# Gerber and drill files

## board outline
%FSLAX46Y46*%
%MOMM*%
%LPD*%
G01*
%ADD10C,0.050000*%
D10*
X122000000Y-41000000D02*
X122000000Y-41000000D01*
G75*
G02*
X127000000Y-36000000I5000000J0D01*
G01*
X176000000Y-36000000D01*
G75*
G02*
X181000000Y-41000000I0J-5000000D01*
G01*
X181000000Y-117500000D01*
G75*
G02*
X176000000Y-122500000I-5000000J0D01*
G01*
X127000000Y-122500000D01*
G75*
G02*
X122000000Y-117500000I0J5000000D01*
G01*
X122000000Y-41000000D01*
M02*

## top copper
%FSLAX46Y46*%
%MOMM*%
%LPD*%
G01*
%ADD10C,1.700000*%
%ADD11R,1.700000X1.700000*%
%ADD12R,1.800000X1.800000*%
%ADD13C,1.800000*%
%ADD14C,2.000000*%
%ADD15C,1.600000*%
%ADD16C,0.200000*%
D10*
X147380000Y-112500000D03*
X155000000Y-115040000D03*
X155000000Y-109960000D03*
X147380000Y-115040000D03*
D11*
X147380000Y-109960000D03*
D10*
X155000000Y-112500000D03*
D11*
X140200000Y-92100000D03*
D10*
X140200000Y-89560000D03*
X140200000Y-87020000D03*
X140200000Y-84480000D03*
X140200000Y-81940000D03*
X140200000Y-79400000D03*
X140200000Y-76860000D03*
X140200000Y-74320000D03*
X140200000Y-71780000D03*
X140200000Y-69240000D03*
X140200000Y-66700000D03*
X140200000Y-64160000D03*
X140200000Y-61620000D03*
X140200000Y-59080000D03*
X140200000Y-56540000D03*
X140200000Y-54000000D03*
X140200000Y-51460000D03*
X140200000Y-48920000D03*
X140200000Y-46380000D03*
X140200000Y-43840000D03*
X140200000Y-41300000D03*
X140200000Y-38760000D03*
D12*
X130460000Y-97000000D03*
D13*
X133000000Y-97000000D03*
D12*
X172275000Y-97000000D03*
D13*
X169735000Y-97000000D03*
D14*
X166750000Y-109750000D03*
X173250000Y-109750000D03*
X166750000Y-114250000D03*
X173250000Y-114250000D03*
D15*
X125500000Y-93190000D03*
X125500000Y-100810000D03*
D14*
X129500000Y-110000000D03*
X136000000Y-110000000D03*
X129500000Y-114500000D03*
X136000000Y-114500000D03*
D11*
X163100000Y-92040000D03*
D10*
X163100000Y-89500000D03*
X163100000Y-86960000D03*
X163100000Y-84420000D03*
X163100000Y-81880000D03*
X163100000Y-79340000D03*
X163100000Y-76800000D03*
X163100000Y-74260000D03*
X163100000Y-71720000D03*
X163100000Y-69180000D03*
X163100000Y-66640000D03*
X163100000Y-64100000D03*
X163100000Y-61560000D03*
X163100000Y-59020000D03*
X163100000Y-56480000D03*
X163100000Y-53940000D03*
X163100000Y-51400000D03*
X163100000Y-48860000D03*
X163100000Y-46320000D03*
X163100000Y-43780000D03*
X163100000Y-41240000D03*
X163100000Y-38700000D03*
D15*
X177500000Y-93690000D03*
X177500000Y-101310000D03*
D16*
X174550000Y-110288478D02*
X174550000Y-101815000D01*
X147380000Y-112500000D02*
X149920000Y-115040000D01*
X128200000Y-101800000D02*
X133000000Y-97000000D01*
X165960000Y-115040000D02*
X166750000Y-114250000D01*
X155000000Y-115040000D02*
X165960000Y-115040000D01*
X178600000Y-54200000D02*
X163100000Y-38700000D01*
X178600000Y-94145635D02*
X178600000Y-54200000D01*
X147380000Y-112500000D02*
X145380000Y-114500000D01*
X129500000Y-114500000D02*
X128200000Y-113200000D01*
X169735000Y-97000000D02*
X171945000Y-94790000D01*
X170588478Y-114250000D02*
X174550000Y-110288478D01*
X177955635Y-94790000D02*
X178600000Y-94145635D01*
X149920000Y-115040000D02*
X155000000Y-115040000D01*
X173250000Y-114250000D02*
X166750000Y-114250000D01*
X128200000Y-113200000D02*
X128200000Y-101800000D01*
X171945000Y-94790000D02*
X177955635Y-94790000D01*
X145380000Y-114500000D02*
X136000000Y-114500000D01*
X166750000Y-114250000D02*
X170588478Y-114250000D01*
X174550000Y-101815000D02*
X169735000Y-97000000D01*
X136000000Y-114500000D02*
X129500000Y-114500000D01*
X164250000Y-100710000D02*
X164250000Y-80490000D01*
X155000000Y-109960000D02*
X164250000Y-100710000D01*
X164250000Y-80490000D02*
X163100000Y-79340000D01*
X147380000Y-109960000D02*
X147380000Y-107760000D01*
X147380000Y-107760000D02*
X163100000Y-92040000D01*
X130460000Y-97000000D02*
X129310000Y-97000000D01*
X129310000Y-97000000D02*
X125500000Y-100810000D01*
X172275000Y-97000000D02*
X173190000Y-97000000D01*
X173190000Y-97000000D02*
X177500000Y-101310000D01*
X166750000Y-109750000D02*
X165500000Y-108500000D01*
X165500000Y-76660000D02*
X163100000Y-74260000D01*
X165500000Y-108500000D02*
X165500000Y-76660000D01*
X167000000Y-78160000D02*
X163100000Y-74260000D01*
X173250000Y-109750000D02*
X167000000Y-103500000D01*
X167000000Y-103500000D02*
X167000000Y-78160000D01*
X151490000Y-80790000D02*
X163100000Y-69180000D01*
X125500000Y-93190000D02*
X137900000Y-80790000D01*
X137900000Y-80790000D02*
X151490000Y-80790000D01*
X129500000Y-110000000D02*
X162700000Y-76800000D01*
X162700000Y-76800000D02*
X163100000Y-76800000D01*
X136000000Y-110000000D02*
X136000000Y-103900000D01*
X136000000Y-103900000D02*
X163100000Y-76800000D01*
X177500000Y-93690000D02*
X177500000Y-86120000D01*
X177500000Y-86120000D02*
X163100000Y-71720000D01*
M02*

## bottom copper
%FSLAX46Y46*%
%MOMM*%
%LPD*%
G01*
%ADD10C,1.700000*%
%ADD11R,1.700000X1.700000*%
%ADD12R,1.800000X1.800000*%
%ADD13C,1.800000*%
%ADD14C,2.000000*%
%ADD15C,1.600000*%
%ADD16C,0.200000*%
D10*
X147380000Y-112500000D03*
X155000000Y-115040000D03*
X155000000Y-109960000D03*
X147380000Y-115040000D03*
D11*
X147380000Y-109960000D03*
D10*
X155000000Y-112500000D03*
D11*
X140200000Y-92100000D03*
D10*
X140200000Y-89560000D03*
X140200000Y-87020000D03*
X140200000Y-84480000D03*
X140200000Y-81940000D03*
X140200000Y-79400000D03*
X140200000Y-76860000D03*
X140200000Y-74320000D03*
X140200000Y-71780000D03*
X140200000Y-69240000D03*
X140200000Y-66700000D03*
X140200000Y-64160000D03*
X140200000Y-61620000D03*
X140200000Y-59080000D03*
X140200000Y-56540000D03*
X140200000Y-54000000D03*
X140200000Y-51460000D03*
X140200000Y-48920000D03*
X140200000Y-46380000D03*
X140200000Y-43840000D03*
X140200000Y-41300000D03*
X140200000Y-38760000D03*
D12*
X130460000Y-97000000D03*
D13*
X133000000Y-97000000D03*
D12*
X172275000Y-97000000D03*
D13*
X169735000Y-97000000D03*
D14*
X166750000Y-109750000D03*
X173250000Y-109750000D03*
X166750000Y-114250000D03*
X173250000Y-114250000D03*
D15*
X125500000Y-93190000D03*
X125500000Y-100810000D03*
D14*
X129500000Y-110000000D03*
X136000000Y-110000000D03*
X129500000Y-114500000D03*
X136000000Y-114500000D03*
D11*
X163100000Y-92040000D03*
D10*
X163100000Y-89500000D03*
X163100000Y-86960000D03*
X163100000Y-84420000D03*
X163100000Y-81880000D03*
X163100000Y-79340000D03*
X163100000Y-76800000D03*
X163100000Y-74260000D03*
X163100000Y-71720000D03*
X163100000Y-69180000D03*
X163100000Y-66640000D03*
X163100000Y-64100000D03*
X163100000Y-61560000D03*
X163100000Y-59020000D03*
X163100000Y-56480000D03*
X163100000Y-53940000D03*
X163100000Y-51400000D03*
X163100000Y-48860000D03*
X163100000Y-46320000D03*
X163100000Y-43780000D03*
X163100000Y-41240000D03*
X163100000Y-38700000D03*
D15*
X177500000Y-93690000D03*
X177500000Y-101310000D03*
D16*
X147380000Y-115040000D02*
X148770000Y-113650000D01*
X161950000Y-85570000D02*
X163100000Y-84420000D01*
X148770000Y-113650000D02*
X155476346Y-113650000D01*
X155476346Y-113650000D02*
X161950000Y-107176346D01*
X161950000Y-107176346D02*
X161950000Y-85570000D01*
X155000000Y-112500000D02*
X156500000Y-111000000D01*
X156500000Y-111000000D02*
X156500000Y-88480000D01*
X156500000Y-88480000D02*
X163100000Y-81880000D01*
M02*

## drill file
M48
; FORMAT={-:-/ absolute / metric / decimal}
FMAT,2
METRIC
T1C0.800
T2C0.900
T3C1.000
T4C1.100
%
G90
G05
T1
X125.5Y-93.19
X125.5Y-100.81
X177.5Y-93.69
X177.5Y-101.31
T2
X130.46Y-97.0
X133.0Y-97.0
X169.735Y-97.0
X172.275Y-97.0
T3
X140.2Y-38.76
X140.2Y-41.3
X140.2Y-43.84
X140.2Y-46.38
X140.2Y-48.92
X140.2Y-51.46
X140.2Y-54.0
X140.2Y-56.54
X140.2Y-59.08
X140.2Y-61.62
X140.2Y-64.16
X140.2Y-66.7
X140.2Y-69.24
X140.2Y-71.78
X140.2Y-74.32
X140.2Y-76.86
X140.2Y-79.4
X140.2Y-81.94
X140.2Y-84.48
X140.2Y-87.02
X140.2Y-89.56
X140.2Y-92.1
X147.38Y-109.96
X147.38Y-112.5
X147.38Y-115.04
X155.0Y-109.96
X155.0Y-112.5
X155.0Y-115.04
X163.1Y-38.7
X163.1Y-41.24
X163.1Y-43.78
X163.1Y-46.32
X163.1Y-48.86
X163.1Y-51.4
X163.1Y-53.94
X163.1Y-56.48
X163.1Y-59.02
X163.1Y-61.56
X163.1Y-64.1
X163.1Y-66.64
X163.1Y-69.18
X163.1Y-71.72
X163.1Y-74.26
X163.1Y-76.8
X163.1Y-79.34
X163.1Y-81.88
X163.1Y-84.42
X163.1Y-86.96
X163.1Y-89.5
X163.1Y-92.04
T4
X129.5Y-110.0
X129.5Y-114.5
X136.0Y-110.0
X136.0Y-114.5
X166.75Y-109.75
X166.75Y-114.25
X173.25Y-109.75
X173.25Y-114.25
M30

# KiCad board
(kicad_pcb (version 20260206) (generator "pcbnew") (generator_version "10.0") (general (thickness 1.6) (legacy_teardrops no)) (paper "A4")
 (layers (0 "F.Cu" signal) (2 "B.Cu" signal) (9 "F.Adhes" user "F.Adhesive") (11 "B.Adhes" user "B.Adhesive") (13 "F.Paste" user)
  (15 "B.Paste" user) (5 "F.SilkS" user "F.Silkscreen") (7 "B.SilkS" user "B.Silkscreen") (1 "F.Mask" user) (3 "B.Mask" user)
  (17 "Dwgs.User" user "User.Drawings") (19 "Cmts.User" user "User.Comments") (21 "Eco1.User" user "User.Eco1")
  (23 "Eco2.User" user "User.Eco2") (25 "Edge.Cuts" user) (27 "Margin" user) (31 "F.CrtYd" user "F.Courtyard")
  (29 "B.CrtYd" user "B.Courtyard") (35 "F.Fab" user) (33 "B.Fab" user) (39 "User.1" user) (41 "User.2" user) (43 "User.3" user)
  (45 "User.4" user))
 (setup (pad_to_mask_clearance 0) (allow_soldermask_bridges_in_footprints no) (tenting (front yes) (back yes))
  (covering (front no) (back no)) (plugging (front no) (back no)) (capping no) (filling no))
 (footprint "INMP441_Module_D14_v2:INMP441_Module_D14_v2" (layer "F.Cu") (at 151.19 112.5)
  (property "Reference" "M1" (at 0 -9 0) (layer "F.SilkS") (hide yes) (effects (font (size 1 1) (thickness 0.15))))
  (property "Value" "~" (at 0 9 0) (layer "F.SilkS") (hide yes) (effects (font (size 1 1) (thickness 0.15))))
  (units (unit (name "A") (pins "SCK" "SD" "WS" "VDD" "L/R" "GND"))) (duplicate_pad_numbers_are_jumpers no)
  (pad "GND" thru_hole circle (at -3.81 0) (size 1.7 1.7) (drill 1) (layers "*.Cu" "*.Mask" "F.SilkS") (remove_unused_layers no) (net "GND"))
  (pad "L/R" thru_hole circle (at 3.81 2.54) (size 1.7 1.7) (drill 1) (layers "*.Cu" "*.Mask" "F.SilkS") (remove_unused_layers no)
   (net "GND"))
  (pad "SCK" thru_hole circle (at 3.81 -2.54) (size 1.7 1.7) (drill 1) (layers "*.Cu" "*.Mask" "F.SilkS") (remove_unused_layers no)
   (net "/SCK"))
  (pad "SD" thru_hole circle (at -3.81 2.54) (size 1.7 1.7) (drill 1) (layers "*.Cu" "*.Mask" "F.SilkS") (remove_unused_layers no)
   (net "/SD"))
  (pad "VDD" thru_hole rect (at -3.81 -2.54) (size 1.7 1.7) (drill 1) (layers "*.Cu" "*.Mask" "F.SilkS") (remove_unused_layers no)
   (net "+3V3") (thermal_bridge_angle 45))
  (pad "WS" thru_hole circle (at 3.81 0) (size 1.7 1.7) (drill 1) (layers "*.Cu" "*.Mask" "F.SilkS") (remove_unused_layers no) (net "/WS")))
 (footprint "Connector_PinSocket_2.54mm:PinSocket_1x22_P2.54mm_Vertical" (layer "F.Cu") (at 140.2 92.1 180)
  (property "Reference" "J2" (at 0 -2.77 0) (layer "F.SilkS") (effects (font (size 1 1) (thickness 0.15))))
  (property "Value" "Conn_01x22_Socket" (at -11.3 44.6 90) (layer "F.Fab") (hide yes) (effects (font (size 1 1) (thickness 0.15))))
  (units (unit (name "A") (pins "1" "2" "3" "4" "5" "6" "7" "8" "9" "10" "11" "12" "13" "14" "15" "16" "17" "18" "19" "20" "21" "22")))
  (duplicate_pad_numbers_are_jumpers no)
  (pad "1" thru_hole rect (at 0 0 180) (size 1.7 1.7) (drill 1) (layers "*.Cu" "*.Mask") (remove_unused_layers no)
   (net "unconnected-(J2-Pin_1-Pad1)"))
  (pad "2" thru_hole circle (at 0 2.54 180) (size 1.7 1.7) (drill 1) (layers "*.Cu" "*.Mask") (remove_unused_layers no)
   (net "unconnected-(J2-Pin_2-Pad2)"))
  (pad "3" thru_hole circle (at 0 5.08 180) (size 1.7 1.7) (drill 1) (layers "*.Cu" "*.Mask") (remove_unused_layers no)
   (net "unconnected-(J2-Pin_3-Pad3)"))
  (pad "4" thru_hole circle (at 0 7.62 180) (size 1.7 1.7) (drill 1) (layers "*.Cu" "*.Mask") (remove_unused_layers no)
   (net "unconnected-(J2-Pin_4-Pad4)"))
  (pad "5" thru_hole circle (at 0 10.16 180) (size 1.7 1.7) (drill 1) (layers "*.Cu" "*.Mask") (remove_unused_layers no)
   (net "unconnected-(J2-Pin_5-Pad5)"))
  (pad "6" thru_hole circle (at 0 12.7 180) (size 1.7 1.7) (drill 1) (layers "*.Cu" "*.Mask") (remove_unused_layers no)
   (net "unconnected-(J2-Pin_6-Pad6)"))
  (pad "7" thru_hole circle (at 0 15.24 180) (size 1.7 1.7) (drill 1) (layers "*.Cu" "*.Mask") (remove_unused_layers no)
   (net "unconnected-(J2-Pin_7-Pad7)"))
  (pad "8" thru_hole circle (at 0 17.78 180) (size 1.7 1.7) (drill 1) (layers "*.Cu" "*.Mask") (remove_unused_layers no)
   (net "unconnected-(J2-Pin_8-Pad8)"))
  (pad "9" thru_hole circle (at 0 20.32 180) (size 1.7 1.7) (drill 1) (layers "*.Cu" "*.Mask") (remove_unused_layers no)
   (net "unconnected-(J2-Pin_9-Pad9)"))
  (pad "10" thru_hole circle (at 0 22.86 180) (size 1.7 1.7) (drill 1) (layers "*.Cu" "*.Mask") (remove_unused_layers no)
   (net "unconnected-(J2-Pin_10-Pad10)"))
  (pad "11" thru_hole circle (at 0 25.4 180) (size 1.7 1.7) (drill 1) (layers "*.Cu" "*.Mask") (remove_unused_layers no)
   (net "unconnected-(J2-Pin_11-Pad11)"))
  (pad "12" thru_hole circle (at 0 27.94 180) (size 1.7 1.7) (drill 1) (layers "*.Cu" "*.Mask") (remove_unused_layers no)
   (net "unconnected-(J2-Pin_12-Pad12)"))
  (pad "13" thru_hole circle (at 0 30.48 180) (size 1.7 1.7) (drill 1) (layers "*.Cu" "*.Mask") (remove_unused_layers no)
   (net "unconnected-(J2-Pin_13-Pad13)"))
  (pad "14" thru_hole circle (at 0 33.02 180) (size 1.7 1.7) (drill 1) (layers "*.Cu" "*.Mask") (remove_unused_layers no)
   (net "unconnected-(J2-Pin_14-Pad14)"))
  (pad "15" thru_hole circle (at 0 35.56 180) (size 1.7 1.7) (drill 1) (layers "*.Cu" "*.Mask") (remove_unused_layers no)
   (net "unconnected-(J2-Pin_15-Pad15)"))
  (pad "16" thru_hole circle (at 0 38.1 180) (size 1.7 1.7) (drill 1) (layers "*.Cu" "*.Mask") (remove_unused_layers no)
   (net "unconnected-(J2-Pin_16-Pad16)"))
  (pad "17" thru_hole circle (at 0 40.64 180) (size 1.7 1.7) (drill 1) (layers "*.Cu" "*.Mask") (remove_unused_layers no)
   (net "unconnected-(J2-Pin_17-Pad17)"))
  (pad "18" thru_hole circle (at 0 43.18 180) (size 1.7 1.7) (drill 1) (layers "*.Cu" "*.Mask") (remove_unused_layers no)
   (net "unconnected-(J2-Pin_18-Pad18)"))
  (pad "19" thru_hole circle (at 0 45.72 180) (size 1.7 1.7) (drill 1) (layers "*.Cu" "*.Mask") (remove_unused_layers no)
   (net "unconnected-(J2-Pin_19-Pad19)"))
  (pad "20" thru_hole circle (at 0 48.26 180) (size 1.7 1.7) (drill 1) (layers "*.Cu" "*.Mask") (remove_unused_layers no)
   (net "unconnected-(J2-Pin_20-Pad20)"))
  (pad "21" thru_hole circle (at 0 50.8 180) (size 1.7 1.7) (drill 1) (layers "*.Cu" "*.Mask") (remove_unused_layers no)
   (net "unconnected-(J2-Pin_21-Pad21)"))
  (pad "22" thru_hole circle (at 0 53.34 180) (size 1.7 1.7) (drill 1) (layers "*.Cu" "*.Mask") (remove_unused_layers no)
   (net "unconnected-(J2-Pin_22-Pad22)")))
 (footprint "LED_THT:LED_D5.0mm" (layer "F.Cu") (at 130.46 97)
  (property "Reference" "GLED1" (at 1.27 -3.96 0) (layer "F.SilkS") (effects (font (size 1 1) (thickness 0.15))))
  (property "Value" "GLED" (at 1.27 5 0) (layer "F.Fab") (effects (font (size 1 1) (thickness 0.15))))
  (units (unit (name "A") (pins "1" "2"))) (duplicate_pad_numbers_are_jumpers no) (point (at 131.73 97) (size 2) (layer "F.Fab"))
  (pad "1" thru_hole rect (at 0 0) (size 1.8 1.8) (drill 0.9) (layers "*.Cu" "*.Mask") (remove_unused_layers no) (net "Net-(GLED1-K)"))
  (pad "2" thru_hole circle (at 2.54 0) (size 1.8 1.8) (drill 0.9) (layers "*.Cu" "*.Mask") (remove_unused_layers no) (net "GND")))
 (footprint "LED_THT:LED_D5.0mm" (layer "F.Cu") (at 172.275 97 180)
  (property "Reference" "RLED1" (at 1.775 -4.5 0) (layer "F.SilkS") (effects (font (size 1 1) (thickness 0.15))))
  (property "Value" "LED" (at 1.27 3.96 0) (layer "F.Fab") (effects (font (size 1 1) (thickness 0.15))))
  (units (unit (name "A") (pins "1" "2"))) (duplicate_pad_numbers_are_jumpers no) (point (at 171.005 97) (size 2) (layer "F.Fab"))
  (pad "1" thru_hole rect (at 0 0 180) (size 1.8 1.8) (drill 0.9) (layers "*.Cu" "*.Mask") (remove_unused_layers no) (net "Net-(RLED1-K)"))
  (pad "2" thru_hole circle (at 2.54 0 180) (size 1.8 1.8) (drill 0.9) (layers "*.Cu" "*.Mask") (remove_unused_layers no) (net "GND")))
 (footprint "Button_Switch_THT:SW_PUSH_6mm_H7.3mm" (layer "F.Cu") (at 166.75 109.75)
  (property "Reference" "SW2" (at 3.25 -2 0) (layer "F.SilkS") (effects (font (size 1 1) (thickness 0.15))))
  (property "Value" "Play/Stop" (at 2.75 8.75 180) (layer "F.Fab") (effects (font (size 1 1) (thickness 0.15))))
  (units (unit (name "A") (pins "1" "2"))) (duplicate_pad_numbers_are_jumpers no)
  (pad "1" thru_hole circle (at 0 0 90) (size 2 2) (drill 1.1) (layers "*.Cu" "*.Mask") (remove_unused_layers no)
   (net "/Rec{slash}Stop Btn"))
  (pad "1" thru_hole circle (at 6.5 0 90) (size 2 2) (drill 1.1) (layers "*.Cu" "*.Mask") (remove_unused_layers no)
   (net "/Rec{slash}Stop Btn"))
  (pad "2" thru_hole circle (at 0 4.5 90) (size 2 2) (drill 1.1) (layers "*.Cu" "*.Mask") (remove_unused_layers no) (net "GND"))
  (pad "2" thru_hole circle (at 6.5 4.5 90) (size 2 2) (drill 1.1) (layers "*.Cu" "*.Mask") (remove_unused_layers no) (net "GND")))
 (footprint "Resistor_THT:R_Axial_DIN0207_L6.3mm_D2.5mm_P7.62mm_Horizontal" (layer "F.Cu") (at 125.5 93.19 -90)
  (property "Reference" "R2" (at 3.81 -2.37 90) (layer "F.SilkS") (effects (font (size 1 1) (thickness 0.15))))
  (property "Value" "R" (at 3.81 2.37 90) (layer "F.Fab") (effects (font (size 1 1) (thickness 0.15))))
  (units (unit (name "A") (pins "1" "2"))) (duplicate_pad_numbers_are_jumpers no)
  (pad "1" thru_hole circle (at 0 0 270) (size 1.6 1.6) (drill 0.8) (layers "*.Cu" "*.Mask") (remove_unused_layers no) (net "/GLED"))
  (pad "2" thru_hole circle (at 7.62 0 270) (size 1.6 1.6) (drill 0.8) (layers "*.Cu" "*.Mask") (remove_unused_layers no)
   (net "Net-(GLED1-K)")))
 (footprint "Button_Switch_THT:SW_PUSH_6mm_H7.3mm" (layer "F.Cu") (at 129.5 110)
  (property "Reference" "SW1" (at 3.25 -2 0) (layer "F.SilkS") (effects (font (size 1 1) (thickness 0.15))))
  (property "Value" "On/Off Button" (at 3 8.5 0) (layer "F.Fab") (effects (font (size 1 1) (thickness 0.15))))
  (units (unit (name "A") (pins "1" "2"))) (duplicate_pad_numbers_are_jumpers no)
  (pad "1" thru_hole circle (at 0 0 90) (size 2 2) (drill 1.1) (layers "*.Cu" "*.Mask") (remove_unused_layers no) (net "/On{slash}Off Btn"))
  (pad "1" thru_hole circle (at 6.5 0 90) (size 2 2) (drill 1.1) (layers "*.Cu" "*.Mask") (remove_unused_layers no)
   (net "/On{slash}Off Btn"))
  (pad "2" thru_hole circle (at 0 4.5 90) (size 2 2) (drill 1.1) (layers "*.Cu" "*.Mask") (remove_unused_layers no) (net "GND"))
  (pad "2" thru_hole circle (at 6.5 4.5 90) (size 2 2) (drill 1.1) (layers "*.Cu" "*.Mask") (remove_unused_layers no) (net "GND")))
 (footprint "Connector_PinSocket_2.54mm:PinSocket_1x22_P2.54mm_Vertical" (layer "F.Cu") (at 163.1 92.04 180)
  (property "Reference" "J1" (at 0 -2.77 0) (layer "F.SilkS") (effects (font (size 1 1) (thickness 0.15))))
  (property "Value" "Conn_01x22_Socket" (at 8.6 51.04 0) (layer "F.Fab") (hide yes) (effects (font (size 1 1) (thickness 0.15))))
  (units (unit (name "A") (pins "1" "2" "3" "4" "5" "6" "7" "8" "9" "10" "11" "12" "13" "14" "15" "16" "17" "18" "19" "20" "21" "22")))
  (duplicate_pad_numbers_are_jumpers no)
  (pad "1" thru_hole rect (at 0 0 180) (size 1.7 1.7) (drill 1) (layers "*.Cu" "*.Mask") (remove_unused_layers no) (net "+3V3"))
  (pad "2" thru_hole circle (at 0 2.54 180) (size 1.7 1.7) (drill 1) (layers "*.Cu" "*.Mask") (remove_unused_layers no)
   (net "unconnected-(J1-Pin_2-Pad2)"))
  (pad "3" thru_hole circle (at 0 5.08 180) (size 1.7 1.7) (drill 1) (layers "*.Cu" "*.Mask") (remove_unused_layers no)
   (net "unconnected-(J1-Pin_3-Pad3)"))
  (pad "4" thru_hole circle (at 0 7.62 180) (size 1.7 1.7) (drill 1) (layers "*.Cu" "*.Mask") (remove_unused_layers no) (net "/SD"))
  (pad "5" thru_hole circle (at 0 10.16 180) (size 1.7 1.7) (drill 1) (layers "*.Cu" "*.Mask") (remove_unused_layers no) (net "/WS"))
  (pad "6" thru_hole circle (at 0 12.7 180) (size 1.7 1.7) (drill 1) (layers "*.Cu" "*.Mask") (remove_unused_layers no) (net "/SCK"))
  (pad "7" thru_hole circle (at 0 15.24 180) (size 1.7 1.7) (drill 1) (layers "*.Cu" "*.Mask") (remove_unused_layers no)
   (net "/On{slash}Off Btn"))
  (pad "8" thru_hole circle (at 0 17.78 180) (size 1.7 1.7) (drill 1) (layers "*.Cu" "*.Mask") (remove_unused_layers no)
   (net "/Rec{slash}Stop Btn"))
  (pad "9" thru_hole circle (at 0 20.32 180) (size 1.7 1.7) (drill 1) (layers "*.Cu" "*.Mask") (remove_unused_layers no) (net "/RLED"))
  (pad "10" thru_hole circle (at 0 22.86 180) (size 1.7 1.7) (drill 1) (layers "*.Cu" "*.Mask") (remove_unused_layers no) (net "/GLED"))
  (pad "11" thru_hole circle (at 0 25.4 180) (size 1.7 1.7) (drill 1) (layers "*.Cu" "*.Mask") (remove_unused_layers no)
   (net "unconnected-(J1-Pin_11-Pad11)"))
  (pad "12" thru_hole circle (at 0 27.94 180) (size 1.7 1.7) (drill 1) (layers "*.Cu" "*.Mask") (remove_unused_layers no)
   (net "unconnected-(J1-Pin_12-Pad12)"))
  (pad "13" thru_hole circle (at 0 30.48 180) (size 1.7 1.7) (drill 1) (layers "*.Cu" "*.Mask") (remove_unused_layers no)
   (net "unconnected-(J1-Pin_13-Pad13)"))
  (pad "14" thru_hole circle (at 0 33.02 180) (size 1.7 1.7) (drill 1) (layers "*.Cu" "*.Mask") (remove_unused_layers no)
   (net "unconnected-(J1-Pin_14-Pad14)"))
  (pad "15" thru_hole circle (at 0 35.56 180) (size 1.7 1.7) (drill 1) (layers "*.Cu" "*.Mask") (remove_unused_layers no)
   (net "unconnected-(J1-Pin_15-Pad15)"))
  (pad "16" thru_hole circle (at 0 38.1 180) (size 1.7 1.7) (drill 1) (layers "*.Cu" "*.Mask") (remove_unused_layers no)
   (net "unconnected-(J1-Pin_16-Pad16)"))
  (pad "17" thru_hole circle (at 0 40.64 180) (size 1.7 1.7) (drill 1) (layers "*.Cu" "*.Mask") (remove_unused_layers no)
   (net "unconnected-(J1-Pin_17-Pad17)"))
  (pad "18" thru_hole circle (at 0 43.18 180) (size 1.7 1.7) (drill 1) (layers "*.Cu" "*.Mask") (remove_unused_layers no)
   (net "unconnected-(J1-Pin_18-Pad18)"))
  (pad "19" thru_hole circle (at 0 45.72 180) (size 1.7 1.7) (drill 1) (layers "*.Cu" "*.Mask") (remove_unused_layers no)
   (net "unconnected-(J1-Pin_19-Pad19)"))
  (pad "20" thru_hole circle (at 0 48.26 180) (size 1.7 1.7) (drill 1) (layers "*.Cu" "*.Mask") (remove_unused_layers no)
   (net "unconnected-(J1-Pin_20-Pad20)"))
  (pad "21" thru_hole circle (at 0 50.8 180) (size 1.7 1.7) (drill 1) (layers "*.Cu" "*.Mask") (remove_unused_layers no)
   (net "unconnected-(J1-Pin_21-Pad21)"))
  (pad "22" thru_hole circle (at 0 53.34 180) (size 1.7 1.7) (drill 1) (layers "*.Cu" "*.Mask") (remove_unused_layers no) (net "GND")))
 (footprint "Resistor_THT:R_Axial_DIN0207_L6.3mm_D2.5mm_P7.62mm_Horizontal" (layer "F.Cu") (at 177.5 93.69 -90)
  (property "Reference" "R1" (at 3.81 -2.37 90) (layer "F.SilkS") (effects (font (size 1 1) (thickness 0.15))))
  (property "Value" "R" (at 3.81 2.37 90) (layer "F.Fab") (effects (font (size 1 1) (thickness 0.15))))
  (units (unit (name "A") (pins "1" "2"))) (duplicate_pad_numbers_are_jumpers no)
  (pad "1" thru_hole circle (at 0 0 270) (size 1.6 1.6) (drill 0.8) (layers "*.Cu" "*.Mask") (remove_unused_layers no) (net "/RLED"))
  (pad "2" thru_hole circle (at 7.62 0 270) (size 1.6 1.6) (drill 0.8) (layers "*.Cu" "*.Mask") (remove_unused_layers no)
   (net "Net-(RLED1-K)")))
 (gr_rect (start 122 36) (end 181 122.5) (radius 5) (stroke (width 0.05) (type solid)) (fill no) (layer "Edge.Cuts"))
 (segment (start 174.55 110.288478) (end 174.55 101.815) (width 0.2) (layer "F.Cu") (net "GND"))
 (segment (start 147.38 112.5) (end 149.92 115.04) (width 0.2) (layer "F.Cu") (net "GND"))
 (segment (start 128.2 101.8) (end 133 97) (width 0.2) (layer "F.Cu") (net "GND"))
 (segment (start 165.96 115.04) (end 166.75 114.25) (width 0.2) (layer "F.Cu") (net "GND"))
 (segment (start 155 115.04) (end 165.96 115.04) (width 0.2) (layer "F.Cu") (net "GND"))
 (segment (start 178.6 54.2) (end 163.1 38.7) (width 0.2) (layer "F.Cu") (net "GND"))
 (segment (start 178.6 94.145635) (end 178.6 54.2) (width 0.2) (layer "F.Cu") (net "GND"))
 (segment (start 147.38 112.5) (end 145.38 114.5) (width 0.2) (layer "F.Cu") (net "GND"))
 (segment (start 129.5 114.5) (end 128.2 113.2) (width 0.2) (layer "F.Cu") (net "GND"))
 (segment (start 169.735 97) (end 171.945 94.79) (width 0.2) (layer "F.Cu") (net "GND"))
 (segment (start 170.588478 114.25) (end 174.55 110.288478) (width 0.2) (layer "F.Cu") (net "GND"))
 (segment (start 177.955635 94.79) (end 178.6 94.145635) (width 0.2) (layer "F.Cu") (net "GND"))
 (segment (start 149.92 115.04) (end 155 115.04) (width 0.2) (layer "F.Cu") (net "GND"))
 (segment (start 173.25 114.25) (end 166.75 114.25) (width 0.2) (layer "F.Cu") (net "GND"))
 (segment (start 128.2 113.2) (end 128.2 101.8) (width 0.2) (layer "F.Cu") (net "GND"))
 (segment (start 171.945 94.79) (end 177.955635 94.79) (width 0.2) (layer "F.Cu") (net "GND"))
 (segment (start 145.38 114.5) (end 136 114.5) (width 0.2) (layer "F.Cu") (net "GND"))
 (segment (start 166.75 114.25) (end 170.588478 114.25) (width 0.2) (layer "F.Cu") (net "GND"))
 (segment (start 174.55 101.815) (end 169.735 97) (width 0.2) (layer "F.Cu") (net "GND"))
 (segment (start 136 114.5) (end 129.5 114.5) (width 0.2) (layer "F.Cu") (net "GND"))
 (segment (start 164.25 100.71) (end 164.25 80.49) (width 0.2) (layer "F.Cu") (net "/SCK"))
 (segment (start 155 109.96) (end 164.25 100.71) (width 0.2) (layer "F.Cu") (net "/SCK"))
 (segment (start 164.25 80.49) (end 163.1 79.34) (width 0.2) (layer "F.Cu") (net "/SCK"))
 (segment (start 147.38 115.04) (end 148.77 113.65) (width 0.2) (layer "B.Cu") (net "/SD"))
 (segment (start 161.95 85.57) (end 163.1 84.42) (width 0.2) (layer "B.Cu") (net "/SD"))
 (segment (start 148.77 113.65) (end 155.476346 113.65) (width 0.2) (layer "B.Cu") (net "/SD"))
 (segment (start 155.476346 113.65) (end 161.95 107.176346) (width 0.2) (layer "B.Cu") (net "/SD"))
 (segment (start 161.95 107.176346) (end 161.95 85.57) (width 0.2) (layer "B.Cu") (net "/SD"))
 (segment (start 147.38 109.96) (end 147.38 107.76) (width 0.2) (layer "F.Cu") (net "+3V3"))
 (segment (start 147.38 107.76) (end 163.1 92.04) (width 0.2) (layer "F.Cu") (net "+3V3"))
 (segment (start 155 112.5) (end 156.5 111) (width 0.2) (layer "B.Cu") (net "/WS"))
 (segment (start 156.5 111) (end 156.5 88.48) (width 0.2) (layer "B.Cu") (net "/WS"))
 (segment (start 156.5 88.48) (end 163.1 81.88) (width 0.2) (layer "B.Cu") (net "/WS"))
 (segment (start 130.46 97) (end 129.31 97) (width 0.2) (layer "F.Cu") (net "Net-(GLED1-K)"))
 (segment (start 129.31 97) (end 125.5 100.81) (width 0.2) (layer "F.Cu") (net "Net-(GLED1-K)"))
 (segment (start 172.275 97) (end 173.19 97) (width 0.2) (layer "F.Cu") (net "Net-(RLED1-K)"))
 (segment (start 173.19 97) (end 177.5 101.31) (width 0.2) (layer "F.Cu") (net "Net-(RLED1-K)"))
 (segment (start 166.75 109.75) (end 165.5 108.5) (width 0.2) (layer "F.Cu") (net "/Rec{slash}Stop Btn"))
 (segment (start 165.5 76.66) (end 163.1 74.26) (width 0.2) (layer "F.Cu") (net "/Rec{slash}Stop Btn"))
 (segment (start 165.5 108.5) (end 165.5 76.66) (width 0.2) (layer "F.Cu") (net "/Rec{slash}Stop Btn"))
 (segment (start 167 78.16) (end 163.1 74.26) (width 0.2) (layer "F.Cu") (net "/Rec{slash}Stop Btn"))
 (segment (start 173.25 109.75) (end 167 103.5) (width 0.2) (layer "F.Cu") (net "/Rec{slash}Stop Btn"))
 (segment (start 167 103.5) (end 167 78.16) (width 0.2) (layer "F.Cu") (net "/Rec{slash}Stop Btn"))
 (segment (start 151.49 80.79) (end 163.1 69.18) (width 0.2) (layer "F.Cu") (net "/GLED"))
 (segment (start 125.5 93.19) (end 137.9 80.79) (width 0.2) (layer "F.Cu") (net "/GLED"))
 (segment (start 137.9 80.79) (end 151.49 80.79) (width 0.2) (layer "F.Cu") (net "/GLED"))
 (segment (start 129.5 110) (end 162.7 76.8) (width 0.2) (layer "F.Cu") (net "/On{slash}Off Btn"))
 (segment (start 162.7 76.8) (end 163.1 76.8) (width 0.2) (layer "F.Cu") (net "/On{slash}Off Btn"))
 (segment (start 136 110) (end 136 103.9) (width 0.2) (layer "F.Cu") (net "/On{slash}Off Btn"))
 (segment (start 136 103.9) (end 163.1 76.8) (width 0.2) (layer "F.Cu") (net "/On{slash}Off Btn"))
 (segment (start 177.5 93.69) (end 177.5 86.12) (width 0.2) (layer "F.Cu") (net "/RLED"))
 (segment (start 177.5 86.12) (end 163.1 71.72) (width 0.2) (layer "F.Cu") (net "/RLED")))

